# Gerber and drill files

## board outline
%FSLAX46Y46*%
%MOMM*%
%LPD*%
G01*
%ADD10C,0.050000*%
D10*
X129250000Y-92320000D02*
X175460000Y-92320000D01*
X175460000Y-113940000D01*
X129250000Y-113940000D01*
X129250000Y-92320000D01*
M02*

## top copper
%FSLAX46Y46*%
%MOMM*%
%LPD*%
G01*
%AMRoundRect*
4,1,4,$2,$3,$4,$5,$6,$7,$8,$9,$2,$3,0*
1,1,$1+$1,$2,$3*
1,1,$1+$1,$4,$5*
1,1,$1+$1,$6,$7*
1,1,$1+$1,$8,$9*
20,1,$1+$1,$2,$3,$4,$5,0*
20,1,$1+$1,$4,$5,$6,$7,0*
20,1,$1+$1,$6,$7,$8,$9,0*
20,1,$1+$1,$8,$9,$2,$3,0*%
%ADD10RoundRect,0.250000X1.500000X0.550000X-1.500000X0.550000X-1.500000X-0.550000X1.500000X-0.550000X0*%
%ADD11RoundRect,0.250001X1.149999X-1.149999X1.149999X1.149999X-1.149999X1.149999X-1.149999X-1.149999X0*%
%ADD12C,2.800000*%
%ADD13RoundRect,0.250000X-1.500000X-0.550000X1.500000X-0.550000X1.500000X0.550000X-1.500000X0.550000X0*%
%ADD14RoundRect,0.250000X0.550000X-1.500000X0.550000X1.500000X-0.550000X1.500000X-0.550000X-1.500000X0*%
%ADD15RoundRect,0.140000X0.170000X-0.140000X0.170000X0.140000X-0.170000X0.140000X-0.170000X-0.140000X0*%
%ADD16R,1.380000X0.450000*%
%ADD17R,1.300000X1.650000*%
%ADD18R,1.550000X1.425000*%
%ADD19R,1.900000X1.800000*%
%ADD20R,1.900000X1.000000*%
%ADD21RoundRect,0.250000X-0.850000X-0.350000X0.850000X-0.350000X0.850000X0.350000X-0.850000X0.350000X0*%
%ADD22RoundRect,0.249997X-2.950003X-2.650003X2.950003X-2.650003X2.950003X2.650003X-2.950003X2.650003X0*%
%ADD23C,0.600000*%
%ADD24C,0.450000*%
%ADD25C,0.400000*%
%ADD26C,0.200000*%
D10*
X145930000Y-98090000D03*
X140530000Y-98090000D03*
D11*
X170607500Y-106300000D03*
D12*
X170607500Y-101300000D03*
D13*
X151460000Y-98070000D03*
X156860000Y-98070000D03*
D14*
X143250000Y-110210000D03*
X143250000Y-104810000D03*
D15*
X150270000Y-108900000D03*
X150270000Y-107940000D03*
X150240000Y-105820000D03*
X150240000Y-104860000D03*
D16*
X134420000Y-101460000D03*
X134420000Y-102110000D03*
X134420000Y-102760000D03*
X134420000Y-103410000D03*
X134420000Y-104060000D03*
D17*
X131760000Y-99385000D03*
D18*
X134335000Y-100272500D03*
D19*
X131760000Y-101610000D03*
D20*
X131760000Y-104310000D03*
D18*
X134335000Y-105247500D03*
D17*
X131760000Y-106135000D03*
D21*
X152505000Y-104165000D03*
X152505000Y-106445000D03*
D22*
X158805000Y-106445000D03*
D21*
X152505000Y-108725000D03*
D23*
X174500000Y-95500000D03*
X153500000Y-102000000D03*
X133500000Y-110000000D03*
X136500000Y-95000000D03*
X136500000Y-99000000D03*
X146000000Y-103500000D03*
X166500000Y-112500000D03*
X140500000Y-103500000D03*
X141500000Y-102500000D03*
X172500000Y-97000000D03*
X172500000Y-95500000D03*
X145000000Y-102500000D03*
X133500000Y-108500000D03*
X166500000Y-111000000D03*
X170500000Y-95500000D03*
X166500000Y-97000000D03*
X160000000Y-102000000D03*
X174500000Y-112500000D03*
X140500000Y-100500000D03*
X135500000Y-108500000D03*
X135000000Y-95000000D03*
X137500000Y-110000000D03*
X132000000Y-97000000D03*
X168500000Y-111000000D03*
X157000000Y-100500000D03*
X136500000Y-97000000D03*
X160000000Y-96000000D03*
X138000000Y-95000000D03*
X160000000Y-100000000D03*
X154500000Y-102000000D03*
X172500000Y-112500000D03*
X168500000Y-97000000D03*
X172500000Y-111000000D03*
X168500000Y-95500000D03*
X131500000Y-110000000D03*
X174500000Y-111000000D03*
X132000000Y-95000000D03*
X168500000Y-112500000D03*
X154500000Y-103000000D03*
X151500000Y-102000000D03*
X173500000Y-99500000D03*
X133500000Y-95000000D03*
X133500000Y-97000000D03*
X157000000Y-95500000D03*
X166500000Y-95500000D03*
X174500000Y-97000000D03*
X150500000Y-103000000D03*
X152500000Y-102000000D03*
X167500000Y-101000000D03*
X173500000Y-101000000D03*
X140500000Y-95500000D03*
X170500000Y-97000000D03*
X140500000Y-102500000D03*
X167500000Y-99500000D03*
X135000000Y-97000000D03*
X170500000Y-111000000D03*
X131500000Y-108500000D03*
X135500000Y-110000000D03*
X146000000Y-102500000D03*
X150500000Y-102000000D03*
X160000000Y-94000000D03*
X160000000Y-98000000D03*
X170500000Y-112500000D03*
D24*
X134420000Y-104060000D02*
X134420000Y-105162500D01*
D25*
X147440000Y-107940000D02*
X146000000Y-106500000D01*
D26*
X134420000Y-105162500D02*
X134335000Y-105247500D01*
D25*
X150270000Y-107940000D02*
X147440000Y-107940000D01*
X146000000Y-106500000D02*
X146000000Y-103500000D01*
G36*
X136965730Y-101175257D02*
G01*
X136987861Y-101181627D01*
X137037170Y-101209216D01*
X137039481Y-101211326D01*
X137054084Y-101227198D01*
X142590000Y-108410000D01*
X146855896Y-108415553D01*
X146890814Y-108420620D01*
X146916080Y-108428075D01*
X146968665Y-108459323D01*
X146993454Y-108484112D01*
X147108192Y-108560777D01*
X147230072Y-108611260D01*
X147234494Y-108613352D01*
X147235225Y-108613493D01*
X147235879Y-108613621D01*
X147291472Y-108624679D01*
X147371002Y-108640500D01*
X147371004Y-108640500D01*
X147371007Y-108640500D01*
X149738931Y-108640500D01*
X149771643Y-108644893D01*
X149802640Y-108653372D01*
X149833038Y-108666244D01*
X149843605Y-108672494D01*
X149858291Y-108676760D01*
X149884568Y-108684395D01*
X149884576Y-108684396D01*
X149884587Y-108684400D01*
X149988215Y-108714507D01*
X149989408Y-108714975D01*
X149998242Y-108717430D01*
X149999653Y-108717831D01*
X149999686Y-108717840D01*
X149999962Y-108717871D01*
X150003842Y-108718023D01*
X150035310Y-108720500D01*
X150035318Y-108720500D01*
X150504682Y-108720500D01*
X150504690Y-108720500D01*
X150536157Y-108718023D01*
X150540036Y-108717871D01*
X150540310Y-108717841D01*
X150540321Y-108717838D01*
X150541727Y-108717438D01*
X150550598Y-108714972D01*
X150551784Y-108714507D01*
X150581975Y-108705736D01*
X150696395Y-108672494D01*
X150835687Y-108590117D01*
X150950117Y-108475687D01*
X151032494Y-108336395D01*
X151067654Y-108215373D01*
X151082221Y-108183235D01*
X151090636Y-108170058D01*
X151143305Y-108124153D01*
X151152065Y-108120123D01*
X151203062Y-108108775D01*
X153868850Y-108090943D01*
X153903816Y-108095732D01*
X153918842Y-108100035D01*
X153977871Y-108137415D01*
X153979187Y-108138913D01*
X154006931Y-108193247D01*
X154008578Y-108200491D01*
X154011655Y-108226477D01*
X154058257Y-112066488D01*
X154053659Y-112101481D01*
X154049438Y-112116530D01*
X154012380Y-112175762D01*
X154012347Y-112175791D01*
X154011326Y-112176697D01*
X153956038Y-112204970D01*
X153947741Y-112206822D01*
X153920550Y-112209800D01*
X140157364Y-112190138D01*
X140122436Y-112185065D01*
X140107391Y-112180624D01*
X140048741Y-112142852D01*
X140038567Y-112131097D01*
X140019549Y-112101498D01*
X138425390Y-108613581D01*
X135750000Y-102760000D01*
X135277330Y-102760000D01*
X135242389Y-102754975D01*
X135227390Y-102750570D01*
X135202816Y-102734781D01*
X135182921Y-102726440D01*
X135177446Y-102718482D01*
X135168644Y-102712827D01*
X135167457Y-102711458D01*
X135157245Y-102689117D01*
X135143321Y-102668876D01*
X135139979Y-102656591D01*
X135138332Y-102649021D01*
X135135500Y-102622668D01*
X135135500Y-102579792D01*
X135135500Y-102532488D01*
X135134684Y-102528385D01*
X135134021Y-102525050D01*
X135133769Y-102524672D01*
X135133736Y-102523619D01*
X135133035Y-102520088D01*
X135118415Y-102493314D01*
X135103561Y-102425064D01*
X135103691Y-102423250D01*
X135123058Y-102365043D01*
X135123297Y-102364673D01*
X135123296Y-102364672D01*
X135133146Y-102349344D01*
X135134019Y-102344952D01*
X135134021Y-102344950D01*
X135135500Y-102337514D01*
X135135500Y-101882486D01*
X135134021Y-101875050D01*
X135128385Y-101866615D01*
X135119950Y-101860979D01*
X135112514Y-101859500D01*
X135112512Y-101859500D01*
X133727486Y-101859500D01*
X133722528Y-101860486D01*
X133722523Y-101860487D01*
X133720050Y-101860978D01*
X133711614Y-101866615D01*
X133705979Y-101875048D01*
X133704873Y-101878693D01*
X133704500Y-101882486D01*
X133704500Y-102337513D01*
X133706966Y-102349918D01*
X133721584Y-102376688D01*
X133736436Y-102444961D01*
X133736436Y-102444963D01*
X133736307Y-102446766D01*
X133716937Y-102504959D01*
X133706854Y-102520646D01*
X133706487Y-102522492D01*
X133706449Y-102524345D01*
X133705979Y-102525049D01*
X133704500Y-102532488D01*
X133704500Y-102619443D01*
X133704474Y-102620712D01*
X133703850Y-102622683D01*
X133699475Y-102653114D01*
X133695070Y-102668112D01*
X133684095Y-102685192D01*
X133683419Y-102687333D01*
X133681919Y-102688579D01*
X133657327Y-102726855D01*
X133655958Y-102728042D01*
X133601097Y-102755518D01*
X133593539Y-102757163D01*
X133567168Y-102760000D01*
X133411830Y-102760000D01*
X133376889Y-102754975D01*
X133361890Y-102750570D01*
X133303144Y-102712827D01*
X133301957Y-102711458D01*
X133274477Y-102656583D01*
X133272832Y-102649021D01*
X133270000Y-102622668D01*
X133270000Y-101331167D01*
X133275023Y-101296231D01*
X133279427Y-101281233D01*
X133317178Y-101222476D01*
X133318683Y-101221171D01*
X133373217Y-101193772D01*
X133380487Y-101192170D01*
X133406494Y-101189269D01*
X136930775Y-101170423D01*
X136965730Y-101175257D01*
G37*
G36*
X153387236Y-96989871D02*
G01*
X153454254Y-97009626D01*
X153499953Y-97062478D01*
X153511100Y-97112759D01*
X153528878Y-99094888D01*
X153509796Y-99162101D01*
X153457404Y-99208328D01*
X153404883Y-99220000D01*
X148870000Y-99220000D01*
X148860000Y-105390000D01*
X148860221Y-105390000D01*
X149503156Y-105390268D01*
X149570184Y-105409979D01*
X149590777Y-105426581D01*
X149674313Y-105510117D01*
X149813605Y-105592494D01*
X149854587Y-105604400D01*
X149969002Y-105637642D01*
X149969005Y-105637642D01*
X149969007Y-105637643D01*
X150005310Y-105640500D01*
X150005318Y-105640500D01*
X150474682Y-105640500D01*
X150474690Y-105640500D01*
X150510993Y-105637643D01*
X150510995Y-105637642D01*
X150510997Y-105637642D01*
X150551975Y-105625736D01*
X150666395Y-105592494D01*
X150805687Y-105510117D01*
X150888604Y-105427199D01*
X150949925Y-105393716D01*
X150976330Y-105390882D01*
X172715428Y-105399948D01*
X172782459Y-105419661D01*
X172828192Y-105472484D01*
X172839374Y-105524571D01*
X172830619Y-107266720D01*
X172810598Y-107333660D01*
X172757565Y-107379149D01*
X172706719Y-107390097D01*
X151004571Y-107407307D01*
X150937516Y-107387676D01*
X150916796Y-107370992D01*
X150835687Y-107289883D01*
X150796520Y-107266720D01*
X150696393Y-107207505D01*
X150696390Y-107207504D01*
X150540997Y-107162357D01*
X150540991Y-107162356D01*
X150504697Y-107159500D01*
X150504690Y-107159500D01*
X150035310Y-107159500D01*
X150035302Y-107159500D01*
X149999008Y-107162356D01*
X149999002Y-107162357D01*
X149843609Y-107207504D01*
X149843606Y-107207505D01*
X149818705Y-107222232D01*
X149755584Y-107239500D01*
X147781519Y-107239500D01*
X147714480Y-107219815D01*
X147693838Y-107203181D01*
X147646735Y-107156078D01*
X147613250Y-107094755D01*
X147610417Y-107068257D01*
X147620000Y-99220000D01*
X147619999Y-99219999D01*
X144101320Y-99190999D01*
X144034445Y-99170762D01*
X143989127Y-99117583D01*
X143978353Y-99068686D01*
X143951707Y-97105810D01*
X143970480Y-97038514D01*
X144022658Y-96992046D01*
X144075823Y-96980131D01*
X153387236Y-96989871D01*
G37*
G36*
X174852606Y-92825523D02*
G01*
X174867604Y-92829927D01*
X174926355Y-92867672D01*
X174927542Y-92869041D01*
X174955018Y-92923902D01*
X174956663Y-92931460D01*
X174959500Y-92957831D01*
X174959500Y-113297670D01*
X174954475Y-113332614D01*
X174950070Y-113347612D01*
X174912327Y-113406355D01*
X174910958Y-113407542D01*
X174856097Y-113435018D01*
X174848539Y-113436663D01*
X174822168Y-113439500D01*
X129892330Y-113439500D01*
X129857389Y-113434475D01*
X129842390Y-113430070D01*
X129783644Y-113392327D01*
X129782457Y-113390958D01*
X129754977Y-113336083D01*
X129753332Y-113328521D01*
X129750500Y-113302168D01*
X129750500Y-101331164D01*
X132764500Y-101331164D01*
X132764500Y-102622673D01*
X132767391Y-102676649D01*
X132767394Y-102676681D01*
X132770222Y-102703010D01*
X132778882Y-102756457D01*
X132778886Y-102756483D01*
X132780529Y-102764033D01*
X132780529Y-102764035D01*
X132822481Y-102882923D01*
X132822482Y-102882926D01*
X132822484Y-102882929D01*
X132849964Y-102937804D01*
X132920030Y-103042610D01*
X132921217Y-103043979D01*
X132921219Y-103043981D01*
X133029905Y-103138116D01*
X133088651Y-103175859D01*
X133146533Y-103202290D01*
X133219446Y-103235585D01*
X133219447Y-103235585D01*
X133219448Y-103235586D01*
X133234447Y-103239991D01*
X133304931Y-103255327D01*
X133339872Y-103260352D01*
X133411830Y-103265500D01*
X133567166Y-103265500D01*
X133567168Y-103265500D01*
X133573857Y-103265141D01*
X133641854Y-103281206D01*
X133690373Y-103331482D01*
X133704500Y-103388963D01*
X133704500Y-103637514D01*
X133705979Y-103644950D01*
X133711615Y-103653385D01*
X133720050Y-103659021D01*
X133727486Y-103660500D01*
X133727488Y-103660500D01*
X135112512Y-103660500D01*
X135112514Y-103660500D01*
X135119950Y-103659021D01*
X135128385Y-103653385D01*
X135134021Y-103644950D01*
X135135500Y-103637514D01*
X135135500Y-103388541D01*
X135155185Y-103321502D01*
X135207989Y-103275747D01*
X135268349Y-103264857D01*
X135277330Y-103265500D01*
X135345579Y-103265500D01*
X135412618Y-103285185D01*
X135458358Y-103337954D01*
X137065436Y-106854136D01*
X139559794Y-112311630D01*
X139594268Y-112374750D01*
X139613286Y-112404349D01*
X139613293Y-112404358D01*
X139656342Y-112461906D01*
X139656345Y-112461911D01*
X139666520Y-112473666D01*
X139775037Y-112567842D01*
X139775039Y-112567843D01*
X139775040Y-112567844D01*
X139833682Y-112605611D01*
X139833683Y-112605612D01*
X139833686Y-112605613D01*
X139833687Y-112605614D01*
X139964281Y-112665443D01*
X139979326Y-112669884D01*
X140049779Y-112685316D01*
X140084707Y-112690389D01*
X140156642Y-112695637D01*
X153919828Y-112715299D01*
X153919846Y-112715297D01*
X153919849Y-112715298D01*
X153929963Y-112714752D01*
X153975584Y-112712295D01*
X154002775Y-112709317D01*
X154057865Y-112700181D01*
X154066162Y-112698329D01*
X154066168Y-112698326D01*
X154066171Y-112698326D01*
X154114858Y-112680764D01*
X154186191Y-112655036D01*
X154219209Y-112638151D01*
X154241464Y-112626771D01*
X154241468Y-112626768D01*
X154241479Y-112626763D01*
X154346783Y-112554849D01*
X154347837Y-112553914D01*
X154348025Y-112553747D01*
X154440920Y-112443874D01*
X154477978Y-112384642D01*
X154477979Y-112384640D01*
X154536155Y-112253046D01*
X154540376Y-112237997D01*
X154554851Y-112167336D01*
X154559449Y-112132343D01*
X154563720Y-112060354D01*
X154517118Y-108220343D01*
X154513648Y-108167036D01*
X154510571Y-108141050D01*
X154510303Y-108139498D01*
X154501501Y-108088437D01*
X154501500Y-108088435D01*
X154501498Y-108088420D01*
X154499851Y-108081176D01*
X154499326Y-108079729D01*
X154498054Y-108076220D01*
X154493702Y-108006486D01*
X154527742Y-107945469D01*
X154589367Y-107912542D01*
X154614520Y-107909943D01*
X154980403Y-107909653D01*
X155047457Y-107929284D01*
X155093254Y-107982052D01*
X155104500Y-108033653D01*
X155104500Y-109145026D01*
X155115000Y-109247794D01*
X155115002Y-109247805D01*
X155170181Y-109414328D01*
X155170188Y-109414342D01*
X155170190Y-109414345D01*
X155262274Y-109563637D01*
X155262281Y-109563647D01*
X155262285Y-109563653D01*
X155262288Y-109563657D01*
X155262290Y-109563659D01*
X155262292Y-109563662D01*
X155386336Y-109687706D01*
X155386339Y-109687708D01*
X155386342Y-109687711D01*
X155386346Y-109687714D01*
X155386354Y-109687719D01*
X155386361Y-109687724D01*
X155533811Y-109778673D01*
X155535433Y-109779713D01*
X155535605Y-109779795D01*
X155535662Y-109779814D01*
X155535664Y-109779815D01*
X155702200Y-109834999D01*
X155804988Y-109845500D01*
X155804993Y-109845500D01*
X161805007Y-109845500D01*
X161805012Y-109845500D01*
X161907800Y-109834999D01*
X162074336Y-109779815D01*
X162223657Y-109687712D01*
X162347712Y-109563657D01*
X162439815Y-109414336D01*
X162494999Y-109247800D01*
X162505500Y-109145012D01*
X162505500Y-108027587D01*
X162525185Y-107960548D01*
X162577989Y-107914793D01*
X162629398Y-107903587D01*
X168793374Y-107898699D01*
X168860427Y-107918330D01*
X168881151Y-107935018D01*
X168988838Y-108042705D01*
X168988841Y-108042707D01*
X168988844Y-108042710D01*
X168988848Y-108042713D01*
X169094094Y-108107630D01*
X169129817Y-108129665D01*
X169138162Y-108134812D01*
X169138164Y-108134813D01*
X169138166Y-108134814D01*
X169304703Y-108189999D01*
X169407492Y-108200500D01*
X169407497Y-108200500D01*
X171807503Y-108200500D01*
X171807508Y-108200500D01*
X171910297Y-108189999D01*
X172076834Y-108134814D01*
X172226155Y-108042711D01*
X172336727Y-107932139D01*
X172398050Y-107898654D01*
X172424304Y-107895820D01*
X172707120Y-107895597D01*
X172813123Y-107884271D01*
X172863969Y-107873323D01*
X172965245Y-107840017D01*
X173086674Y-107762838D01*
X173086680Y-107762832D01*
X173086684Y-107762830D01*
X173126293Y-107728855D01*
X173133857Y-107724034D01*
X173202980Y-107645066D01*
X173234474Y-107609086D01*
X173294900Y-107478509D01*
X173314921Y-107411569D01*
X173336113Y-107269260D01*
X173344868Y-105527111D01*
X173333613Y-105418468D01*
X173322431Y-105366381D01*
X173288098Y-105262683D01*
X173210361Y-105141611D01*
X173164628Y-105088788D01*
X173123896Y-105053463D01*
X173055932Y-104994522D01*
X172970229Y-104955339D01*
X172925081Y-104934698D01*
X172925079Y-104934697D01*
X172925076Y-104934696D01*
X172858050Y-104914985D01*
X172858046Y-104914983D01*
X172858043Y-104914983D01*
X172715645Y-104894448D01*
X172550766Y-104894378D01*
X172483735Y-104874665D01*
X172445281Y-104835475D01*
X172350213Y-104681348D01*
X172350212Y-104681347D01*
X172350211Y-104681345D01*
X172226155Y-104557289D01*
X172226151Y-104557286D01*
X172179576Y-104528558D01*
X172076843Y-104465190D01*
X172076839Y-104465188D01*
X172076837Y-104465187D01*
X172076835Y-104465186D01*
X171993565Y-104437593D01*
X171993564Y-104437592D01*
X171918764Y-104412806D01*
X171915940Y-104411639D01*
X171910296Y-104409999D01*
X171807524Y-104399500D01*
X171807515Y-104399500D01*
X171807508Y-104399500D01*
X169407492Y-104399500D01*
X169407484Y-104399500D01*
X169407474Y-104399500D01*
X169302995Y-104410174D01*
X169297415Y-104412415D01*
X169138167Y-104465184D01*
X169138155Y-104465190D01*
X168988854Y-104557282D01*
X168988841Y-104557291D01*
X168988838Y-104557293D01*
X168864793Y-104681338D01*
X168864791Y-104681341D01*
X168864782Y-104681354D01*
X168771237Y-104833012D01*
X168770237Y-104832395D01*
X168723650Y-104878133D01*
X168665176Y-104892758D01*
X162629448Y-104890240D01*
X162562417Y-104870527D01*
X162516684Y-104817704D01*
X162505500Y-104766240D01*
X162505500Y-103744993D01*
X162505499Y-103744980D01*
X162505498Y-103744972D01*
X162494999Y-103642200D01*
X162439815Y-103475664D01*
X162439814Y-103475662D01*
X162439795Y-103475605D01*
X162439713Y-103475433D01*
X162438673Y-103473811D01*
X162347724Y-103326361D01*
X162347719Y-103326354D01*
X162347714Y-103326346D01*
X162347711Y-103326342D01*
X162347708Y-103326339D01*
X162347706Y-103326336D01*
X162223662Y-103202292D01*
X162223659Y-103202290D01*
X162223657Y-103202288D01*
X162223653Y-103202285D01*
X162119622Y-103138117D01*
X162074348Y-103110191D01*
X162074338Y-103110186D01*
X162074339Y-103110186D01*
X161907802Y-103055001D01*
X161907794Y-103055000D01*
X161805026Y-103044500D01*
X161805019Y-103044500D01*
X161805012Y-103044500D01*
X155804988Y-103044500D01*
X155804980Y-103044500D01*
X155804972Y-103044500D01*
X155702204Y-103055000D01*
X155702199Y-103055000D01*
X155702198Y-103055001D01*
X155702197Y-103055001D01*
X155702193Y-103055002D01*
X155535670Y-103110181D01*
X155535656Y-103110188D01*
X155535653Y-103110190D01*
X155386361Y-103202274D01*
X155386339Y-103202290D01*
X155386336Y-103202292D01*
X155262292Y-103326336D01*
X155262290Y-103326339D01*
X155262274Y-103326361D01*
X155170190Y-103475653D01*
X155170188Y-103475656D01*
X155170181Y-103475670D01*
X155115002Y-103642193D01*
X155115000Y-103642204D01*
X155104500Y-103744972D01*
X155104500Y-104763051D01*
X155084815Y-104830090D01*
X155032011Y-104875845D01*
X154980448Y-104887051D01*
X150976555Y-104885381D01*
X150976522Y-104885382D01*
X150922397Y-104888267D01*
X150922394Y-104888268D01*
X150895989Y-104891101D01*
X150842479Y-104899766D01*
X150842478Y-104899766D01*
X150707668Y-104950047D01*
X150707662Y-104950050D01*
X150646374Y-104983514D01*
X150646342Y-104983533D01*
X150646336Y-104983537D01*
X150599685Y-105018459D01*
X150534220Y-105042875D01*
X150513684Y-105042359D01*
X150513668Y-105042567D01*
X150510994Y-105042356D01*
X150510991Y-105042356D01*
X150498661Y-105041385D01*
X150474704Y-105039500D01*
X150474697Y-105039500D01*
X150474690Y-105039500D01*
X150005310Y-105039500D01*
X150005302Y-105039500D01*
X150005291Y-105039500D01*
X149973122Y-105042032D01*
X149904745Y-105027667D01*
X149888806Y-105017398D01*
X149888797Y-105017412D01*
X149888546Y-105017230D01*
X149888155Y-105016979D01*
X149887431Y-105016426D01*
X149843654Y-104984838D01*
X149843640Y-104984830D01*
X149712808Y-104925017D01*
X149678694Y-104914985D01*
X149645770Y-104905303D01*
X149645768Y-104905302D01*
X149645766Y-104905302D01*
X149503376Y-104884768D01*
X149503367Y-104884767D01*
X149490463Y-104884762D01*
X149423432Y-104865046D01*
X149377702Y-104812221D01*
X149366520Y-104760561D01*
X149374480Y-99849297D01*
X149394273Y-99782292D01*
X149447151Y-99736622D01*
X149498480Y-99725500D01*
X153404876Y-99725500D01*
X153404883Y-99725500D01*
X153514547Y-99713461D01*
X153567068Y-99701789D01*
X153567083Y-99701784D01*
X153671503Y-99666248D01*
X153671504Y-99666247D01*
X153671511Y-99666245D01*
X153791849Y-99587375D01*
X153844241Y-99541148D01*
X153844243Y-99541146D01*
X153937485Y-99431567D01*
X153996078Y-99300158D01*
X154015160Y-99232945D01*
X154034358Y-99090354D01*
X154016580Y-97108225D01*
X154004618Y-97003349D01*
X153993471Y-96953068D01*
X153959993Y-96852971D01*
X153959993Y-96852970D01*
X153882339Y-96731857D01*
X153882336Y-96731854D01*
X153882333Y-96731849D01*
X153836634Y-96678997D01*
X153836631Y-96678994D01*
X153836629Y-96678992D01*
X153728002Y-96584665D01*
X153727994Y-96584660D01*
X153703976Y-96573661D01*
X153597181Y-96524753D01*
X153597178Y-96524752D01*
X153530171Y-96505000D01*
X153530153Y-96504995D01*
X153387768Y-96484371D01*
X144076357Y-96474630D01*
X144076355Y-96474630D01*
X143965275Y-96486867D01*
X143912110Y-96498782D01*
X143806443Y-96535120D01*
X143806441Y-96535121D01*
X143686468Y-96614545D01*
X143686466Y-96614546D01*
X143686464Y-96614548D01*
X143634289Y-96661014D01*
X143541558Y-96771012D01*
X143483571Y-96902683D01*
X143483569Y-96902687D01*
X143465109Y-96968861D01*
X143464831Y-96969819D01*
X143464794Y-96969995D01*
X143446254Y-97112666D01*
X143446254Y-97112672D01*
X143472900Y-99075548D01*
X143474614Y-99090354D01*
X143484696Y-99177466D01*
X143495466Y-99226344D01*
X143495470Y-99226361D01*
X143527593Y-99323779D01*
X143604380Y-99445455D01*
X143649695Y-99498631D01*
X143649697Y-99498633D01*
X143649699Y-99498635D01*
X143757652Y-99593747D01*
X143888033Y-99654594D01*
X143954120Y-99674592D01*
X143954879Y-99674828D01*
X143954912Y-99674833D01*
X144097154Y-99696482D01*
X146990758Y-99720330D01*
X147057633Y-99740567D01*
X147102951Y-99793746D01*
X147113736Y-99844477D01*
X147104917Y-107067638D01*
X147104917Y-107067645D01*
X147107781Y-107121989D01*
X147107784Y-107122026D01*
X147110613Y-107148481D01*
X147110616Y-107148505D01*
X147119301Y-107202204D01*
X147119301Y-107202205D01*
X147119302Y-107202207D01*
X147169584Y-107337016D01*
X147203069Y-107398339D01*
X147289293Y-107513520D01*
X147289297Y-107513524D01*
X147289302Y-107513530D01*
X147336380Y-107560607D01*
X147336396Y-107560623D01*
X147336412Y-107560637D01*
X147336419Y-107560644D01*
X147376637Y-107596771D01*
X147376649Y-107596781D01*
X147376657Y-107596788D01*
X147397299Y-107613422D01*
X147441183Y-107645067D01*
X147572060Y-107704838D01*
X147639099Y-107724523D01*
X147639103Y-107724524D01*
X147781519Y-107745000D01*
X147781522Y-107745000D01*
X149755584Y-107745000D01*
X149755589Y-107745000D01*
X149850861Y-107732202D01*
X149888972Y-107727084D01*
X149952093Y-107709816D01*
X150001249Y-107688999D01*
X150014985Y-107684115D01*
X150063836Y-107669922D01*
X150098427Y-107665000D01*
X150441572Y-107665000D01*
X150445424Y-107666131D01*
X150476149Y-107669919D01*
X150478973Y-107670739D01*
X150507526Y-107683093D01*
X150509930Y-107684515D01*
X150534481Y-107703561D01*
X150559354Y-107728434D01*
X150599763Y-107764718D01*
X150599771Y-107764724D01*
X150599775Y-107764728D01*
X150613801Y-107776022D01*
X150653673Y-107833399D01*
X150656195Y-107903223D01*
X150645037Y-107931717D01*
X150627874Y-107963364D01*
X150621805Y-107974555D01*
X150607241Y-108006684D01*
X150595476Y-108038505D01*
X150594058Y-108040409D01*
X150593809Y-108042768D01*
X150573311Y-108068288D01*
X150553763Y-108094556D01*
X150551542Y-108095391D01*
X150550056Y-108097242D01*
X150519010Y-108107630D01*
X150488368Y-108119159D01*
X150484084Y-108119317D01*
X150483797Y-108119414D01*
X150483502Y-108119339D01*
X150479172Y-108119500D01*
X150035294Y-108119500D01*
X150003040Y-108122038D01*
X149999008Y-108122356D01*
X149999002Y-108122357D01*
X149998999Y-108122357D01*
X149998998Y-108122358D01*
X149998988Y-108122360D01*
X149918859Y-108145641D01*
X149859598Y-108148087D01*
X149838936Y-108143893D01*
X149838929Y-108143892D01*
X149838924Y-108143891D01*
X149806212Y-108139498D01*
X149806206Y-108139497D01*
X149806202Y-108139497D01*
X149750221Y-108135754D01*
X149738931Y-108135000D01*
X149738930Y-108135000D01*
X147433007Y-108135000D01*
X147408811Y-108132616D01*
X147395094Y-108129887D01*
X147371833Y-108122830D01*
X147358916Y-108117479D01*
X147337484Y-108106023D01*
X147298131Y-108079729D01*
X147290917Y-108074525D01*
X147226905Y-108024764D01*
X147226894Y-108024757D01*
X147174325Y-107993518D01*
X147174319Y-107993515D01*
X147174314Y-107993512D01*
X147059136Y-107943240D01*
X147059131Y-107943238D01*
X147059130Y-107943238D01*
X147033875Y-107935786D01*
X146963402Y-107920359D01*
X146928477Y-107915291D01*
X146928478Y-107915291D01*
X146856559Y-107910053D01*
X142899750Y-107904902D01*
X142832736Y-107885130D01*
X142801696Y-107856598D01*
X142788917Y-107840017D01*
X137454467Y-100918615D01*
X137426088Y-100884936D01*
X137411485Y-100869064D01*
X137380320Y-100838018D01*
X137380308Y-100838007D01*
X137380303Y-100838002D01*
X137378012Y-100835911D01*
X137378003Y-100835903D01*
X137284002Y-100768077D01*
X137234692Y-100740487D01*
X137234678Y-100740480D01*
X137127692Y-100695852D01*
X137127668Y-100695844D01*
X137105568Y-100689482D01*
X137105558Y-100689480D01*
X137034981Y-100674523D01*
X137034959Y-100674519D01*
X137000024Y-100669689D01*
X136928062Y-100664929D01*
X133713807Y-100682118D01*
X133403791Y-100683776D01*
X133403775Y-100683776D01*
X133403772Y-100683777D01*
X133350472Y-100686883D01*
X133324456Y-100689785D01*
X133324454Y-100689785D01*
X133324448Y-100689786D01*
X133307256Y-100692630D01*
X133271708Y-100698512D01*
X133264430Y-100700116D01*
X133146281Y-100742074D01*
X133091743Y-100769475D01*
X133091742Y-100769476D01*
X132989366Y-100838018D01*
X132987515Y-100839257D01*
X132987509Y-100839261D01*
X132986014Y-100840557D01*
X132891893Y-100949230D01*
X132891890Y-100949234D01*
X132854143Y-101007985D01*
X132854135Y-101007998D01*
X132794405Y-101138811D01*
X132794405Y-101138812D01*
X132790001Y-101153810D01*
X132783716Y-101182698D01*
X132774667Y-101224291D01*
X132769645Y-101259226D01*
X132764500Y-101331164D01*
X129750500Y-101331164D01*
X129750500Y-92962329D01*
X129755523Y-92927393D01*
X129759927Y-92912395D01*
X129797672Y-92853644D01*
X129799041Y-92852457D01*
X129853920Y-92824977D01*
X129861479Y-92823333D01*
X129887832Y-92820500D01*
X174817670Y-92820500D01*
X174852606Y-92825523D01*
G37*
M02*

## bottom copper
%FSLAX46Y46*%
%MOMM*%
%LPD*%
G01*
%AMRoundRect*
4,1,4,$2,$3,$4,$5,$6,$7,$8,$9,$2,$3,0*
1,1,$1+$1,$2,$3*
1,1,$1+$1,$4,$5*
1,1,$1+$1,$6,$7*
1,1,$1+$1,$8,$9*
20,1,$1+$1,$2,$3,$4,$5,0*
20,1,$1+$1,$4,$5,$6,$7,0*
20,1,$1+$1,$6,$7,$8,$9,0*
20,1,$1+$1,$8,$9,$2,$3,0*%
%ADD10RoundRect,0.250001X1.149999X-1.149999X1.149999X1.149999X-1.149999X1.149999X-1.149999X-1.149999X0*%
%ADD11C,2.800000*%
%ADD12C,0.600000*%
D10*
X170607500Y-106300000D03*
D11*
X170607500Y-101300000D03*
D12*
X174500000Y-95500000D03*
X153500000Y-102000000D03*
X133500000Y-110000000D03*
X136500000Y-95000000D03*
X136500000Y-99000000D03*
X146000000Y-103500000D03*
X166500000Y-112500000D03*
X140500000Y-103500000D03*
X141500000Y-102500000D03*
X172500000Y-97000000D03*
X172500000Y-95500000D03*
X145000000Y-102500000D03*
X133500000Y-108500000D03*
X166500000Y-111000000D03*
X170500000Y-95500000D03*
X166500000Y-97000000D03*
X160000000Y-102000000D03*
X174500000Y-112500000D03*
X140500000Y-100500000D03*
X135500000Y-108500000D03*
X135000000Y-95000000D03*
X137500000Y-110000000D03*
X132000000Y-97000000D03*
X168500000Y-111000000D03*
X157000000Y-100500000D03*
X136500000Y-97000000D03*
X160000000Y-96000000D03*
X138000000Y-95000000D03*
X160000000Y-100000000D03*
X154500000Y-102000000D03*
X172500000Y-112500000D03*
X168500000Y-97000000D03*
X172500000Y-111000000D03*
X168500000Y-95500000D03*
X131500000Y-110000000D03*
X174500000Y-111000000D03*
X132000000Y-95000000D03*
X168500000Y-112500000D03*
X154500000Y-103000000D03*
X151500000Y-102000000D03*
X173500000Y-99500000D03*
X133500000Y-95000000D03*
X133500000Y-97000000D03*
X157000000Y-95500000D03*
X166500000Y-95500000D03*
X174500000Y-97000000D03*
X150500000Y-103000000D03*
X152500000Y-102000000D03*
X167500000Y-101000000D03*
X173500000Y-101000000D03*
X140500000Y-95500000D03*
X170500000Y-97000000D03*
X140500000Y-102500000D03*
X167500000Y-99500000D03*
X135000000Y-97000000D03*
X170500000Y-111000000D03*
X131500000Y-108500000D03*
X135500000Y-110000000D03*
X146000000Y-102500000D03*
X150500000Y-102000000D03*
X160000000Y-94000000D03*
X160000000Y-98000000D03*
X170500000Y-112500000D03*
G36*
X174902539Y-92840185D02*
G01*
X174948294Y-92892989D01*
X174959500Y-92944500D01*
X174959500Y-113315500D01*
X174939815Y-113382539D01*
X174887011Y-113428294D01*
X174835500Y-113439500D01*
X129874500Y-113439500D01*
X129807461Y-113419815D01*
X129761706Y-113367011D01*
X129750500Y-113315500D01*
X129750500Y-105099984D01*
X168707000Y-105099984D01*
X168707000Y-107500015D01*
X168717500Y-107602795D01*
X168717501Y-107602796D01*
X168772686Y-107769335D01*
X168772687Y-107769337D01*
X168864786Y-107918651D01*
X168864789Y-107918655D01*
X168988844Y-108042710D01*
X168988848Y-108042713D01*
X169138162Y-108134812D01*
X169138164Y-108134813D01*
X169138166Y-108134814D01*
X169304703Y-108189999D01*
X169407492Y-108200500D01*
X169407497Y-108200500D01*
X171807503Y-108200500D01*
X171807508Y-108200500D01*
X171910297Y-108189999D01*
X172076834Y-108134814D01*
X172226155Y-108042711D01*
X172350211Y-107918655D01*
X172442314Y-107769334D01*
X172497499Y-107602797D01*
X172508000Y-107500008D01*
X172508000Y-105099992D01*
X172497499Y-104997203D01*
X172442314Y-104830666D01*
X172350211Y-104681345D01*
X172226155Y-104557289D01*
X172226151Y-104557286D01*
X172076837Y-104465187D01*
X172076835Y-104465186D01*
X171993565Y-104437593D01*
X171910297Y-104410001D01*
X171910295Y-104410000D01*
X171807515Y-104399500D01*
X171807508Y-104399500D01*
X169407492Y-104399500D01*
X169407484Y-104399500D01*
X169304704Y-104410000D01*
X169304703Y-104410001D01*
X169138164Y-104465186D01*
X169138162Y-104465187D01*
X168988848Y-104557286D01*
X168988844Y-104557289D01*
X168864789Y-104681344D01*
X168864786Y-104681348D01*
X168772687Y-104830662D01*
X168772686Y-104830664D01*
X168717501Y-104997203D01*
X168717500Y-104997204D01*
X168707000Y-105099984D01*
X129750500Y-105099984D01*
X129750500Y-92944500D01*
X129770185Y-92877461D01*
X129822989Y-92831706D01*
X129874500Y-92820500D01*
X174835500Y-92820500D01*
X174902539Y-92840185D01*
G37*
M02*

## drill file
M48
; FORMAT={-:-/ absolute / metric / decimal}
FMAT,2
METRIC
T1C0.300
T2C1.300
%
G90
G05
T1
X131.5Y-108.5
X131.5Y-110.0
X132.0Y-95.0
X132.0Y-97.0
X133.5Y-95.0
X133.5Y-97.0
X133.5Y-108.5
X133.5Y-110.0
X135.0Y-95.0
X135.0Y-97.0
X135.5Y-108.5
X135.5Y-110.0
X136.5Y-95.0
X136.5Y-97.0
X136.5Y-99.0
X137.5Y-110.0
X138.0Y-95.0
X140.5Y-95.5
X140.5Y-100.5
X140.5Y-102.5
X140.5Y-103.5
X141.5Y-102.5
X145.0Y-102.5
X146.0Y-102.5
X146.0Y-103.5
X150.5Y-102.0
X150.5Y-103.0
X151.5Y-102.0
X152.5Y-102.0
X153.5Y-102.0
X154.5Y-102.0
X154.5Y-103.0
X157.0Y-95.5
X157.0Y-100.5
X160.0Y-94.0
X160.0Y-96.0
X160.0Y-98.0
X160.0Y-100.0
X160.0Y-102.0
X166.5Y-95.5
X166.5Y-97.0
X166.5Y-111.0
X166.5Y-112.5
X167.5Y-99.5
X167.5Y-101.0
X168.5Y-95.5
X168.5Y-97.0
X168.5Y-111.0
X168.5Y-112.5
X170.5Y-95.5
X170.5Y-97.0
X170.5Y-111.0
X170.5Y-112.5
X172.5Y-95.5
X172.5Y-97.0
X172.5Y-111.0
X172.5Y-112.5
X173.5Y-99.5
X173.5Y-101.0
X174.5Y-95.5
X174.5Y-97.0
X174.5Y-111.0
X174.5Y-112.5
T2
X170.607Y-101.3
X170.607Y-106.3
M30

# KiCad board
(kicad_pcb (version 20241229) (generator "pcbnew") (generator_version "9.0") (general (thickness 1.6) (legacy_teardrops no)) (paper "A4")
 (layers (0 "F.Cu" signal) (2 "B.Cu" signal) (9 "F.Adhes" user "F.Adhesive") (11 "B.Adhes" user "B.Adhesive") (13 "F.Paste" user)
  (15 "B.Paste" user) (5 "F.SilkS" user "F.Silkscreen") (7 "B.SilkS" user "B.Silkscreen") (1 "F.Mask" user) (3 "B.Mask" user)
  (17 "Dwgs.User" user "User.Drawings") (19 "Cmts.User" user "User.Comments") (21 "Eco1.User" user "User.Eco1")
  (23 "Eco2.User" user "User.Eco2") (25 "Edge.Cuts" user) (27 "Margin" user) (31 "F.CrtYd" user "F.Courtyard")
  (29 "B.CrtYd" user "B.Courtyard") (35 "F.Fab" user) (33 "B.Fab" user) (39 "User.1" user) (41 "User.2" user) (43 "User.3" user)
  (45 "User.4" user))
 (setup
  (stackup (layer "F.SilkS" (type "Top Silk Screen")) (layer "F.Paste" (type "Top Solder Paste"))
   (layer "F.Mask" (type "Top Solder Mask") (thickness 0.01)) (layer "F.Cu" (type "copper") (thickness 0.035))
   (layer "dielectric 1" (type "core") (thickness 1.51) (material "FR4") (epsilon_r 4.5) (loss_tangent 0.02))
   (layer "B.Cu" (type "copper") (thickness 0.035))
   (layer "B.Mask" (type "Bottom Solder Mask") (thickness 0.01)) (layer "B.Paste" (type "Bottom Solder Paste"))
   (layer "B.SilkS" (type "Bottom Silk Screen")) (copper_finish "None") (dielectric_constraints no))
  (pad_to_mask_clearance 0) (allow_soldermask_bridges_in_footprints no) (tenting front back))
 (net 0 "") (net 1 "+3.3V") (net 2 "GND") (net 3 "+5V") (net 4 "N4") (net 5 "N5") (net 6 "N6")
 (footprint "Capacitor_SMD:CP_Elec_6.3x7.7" (layer "F.Cu") (at 143.23 98.09 180)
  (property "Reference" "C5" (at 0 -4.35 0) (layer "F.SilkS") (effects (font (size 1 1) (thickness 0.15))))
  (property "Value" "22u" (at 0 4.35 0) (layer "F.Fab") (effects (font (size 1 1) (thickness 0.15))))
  (pad "1" smd roundrect (at -2.7 0 180) (size 3.5 1.6) (layers "F.Cu" "F.Mask" "F.Paste") (roundrect_rratio 0.15625) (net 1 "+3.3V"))
  (pad "2" smd roundrect (at 2.7 0 180) (size 3.5 1.6) (layers "F.Cu" "F.Mask" "F.Paste") (roundrect_rratio 0.15625) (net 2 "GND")))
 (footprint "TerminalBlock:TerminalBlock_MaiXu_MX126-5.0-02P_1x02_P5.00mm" (layer "F.Cu") (at 170.6075 106.3 90)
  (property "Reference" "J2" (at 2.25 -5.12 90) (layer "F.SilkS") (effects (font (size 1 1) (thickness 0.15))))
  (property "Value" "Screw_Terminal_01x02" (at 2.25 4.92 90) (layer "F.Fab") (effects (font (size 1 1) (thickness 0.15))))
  (pad "1" thru_hole roundrect (at 0 0 90) (size 2.8 2.8) (drill 1.3) (layers "*.Cu" "*.Mask") (remove_unused_layers no)
   (roundrect_rratio 0.089286) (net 1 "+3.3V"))
  (pad "2" thru_hole circle (at 5 0 90) (size 2.8 2.8) (drill 1.3) (layers "*.Cu" "*.Mask") (remove_unused_layers no) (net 2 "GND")))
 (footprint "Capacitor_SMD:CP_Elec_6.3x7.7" (layer "F.Cu") (at 154.16 98.07)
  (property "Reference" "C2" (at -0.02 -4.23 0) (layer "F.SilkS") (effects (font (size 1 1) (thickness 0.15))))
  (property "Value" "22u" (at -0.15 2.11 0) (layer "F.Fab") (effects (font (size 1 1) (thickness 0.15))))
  (pad "1" smd roundrect (at -2.7 0) (size 3.5 1.6) (layers "F.Cu" "F.Mask" "F.Paste") (roundrect_rratio 0.15625) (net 1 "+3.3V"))
  (pad "2" smd roundrect (at 2.7 0) (size 3.5 1.6) (layers "F.Cu" "F.Mask" "F.Paste") (roundrect_rratio 0.15625) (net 2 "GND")))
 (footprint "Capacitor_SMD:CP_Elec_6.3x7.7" (layer "F.Cu") (at 143.25 107.51 90)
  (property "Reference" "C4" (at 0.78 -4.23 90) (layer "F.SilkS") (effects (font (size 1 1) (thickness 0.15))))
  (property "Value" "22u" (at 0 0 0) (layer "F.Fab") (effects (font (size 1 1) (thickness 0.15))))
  (pad "1" smd roundrect (at -2.7 0 90) (size 3.5 1.6) (layers "F.Cu" "F.Mask" "F.Paste") (roundrect_rratio 0.15625) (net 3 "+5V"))
  (pad "2" smd roundrect (at 2.7 0 90) (size 3.5 1.6) (layers "F.Cu" "F.Mask" "F.Paste") (roundrect_rratio 0.15625) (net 2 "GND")))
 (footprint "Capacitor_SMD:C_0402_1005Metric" (layer "F.Cu") (at 150.27 108.42 90)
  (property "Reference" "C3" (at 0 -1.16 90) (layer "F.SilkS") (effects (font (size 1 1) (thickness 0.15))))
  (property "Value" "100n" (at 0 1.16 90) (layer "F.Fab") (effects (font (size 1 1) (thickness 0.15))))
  (pad "1" smd roundrect (at -0.48 0 90) (size 0.56 0.62) (layers "F.Cu" "F.Mask" "F.Paste") (roundrect_rratio 0.25) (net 3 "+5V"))
  (pad "2" smd roundrect (at 0.48 0 90) (size 0.56 0.62) (layers "F.Cu" "F.Mask" "F.Paste") (roundrect_rratio 0.25) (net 2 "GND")))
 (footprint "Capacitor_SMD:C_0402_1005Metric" (layer "F.Cu") (at 150.24 105.34 90)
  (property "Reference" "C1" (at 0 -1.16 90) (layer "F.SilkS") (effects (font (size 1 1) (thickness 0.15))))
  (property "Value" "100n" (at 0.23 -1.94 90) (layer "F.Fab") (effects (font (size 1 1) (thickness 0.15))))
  (pad "1" smd roundrect (at -0.48 0 90) (size 0.56 0.62) (layers "F.Cu" "F.Mask" "F.Paste") (roundrect_rratio 0.25) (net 1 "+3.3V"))
  (pad "2" smd roundrect (at 0.48 0 90) (size 0.56 0.62) (layers "F.Cu" "F.Mask" "F.Paste") (roundrect_rratio 0.25) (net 2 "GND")))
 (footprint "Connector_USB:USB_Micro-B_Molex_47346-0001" (layer "F.Cu") (at 132.96 102.76 -90)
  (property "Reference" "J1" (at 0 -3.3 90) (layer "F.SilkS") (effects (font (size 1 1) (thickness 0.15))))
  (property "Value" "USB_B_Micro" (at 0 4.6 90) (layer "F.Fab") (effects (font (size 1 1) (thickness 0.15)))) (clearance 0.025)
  (pad "1" smd rect (at -1.3 -1.46 270) (size 0.45 1.38) (layers "F.Cu" "F.Mask" "F.Paste") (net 3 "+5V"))
  (pad "2" smd rect (at -0.65 -1.46 270) (size 0.45 1.38) (layers "F.Cu" "F.Mask" "F.Paste") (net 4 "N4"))
  (pad "3" smd rect (at 0 -1.46 270) (size 0.45 1.38) (layers "F.Cu" "F.Mask" "F.Paste") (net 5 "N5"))
  (pad "4" smd rect (at 0.65 -1.46 270) (size 0.45 1.38) (layers "F.Cu" "F.Mask" "F.Paste") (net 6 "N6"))
  (pad "5" smd rect (at 1.3 -1.46 270) (size 0.45 1.38) (layers "F.Cu" "F.Mask" "F.Paste") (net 2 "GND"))
  (pad "6" smd rect (at -3.375 1.2 270) (size 1.65 1.3) (layers "F.Cu" "F.Mask" "F.Paste") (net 2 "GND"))
  (pad "6" smd rect (at -2.4875 -1.375 270) (size 1.425 1.55) (layers "F.Cu" "F.Mask" "F.Paste") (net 2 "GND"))
  (pad "6" smd rect (at -1.15 1.2 270) (size 1.8 1.9) (layers "F.Cu" "F.Mask" "F.Paste") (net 2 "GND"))
  (pad "6" smd rect (at 1.55 1.2 270) (size 1 1.9) (layers "F.Cu" "F.Mask" "F.Paste") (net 2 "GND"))
  (pad "6" smd rect (at 2.4875 -1.375 270) (size 1.425 1.55) (layers "F.Cu" "F.Mask" "F.Paste") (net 2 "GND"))
  (pad "6" smd rect (at 3.375 1.2 270) (size 1.65 1.3) (layers "F.Cu" "F.Mask" "F.Paste") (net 2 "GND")))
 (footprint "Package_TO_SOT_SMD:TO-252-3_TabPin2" (layer "F.Cu") (at 157.545 106.445)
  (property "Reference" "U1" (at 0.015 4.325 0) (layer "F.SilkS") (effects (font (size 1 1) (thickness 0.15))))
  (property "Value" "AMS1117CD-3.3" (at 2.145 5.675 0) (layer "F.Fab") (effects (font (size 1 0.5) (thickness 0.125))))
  (pad "" smd roundrect (at -0.415 -1.525) (size 3.05 2.75) (layers "F.Paste") (roundrect_rratio 0.090909))
  (pad "" smd roundrect (at -0.415 1.525) (size 3.05 2.75) (layers "F.Paste") (roundrect_rratio 0.090909))
  (pad "" smd roundrect (at 2.935 -1.525) (size 3.05 2.75) (layers "F.Paste") (roundrect_rratio 0.090909))
  (pad "" smd roundrect (at 2.935 1.525) (size 3.05 2.75) (layers "F.Paste") (roundrect_rratio 0.090909))
  (pad "1" smd roundrect (at -5.04 -2.28) (size 2.2 1.2) (layers "F.Cu" "F.Mask" "F.Paste") (roundrect_rratio 0.208333) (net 2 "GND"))
  (pad "2" smd roundrect (at -5.04 0) (size 2.2 1.2) (layers "F.Cu" "F.Mask" "F.Paste") (roundrect_rratio 0.208333) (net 1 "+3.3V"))
  (pad "2" smd roundrect (at 1.26 0) (size 6.4 5.8) (layers "F.Cu" "F.Mask") (roundrect_rratio 0.043103) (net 1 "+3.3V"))
  (pad "3" smd roundrect (at -5.04 2.28) (size 2.2 1.2) (layers "F.Cu" "F.Mask" "F.Paste") (roundrect_rratio 0.208333) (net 3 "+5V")))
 (gr_rect (start 129.25 92.32) (end 175.46 113.94) (stroke (width 0.05) (type default)) (fill no) (layer "Edge.Cuts"))
 (segment (start 134.42 104.06) (end 134.42 105.1625) (width 0.45) (layer "F.Cu") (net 2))
 (segment (start 147.44 107.94) (end 146 106.5) (width 0.4) (layer "F.Cu") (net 2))
 (segment (start 134.42 105.1625) (end 134.335 105.2475) (width 0.2) (layer "F.Cu") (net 2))
 (segment (start 150.27 107.94) (end 147.44 107.94) (width 0.4) (layer "F.Cu") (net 2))
 (segment (start 146 106.5) (end 146 103.5) (width 0.4) (layer "F.Cu") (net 2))
 (via (at 174.5 95.5) (size 0.6) (drill 0.3) (layers "F.Cu" "B.Cu") (free yes) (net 2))
 (via (at 153.5 102) (size 0.6) (drill 0.3) (layers "F.Cu" "B.Cu") (free yes) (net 2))
 (via (at 133.5 110) (size 0.6) (drill 0.3) (layers "F.Cu" "B.Cu") (free yes) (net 2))
 (via (at 136.5 95) (size 0.6) (drill 0.3) (layers "F.Cu" "B.Cu") (free yes) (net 2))
 (via (at 136.5 99) (size 0.6) (drill 0.3) (layers "F.Cu" "B.Cu") (free yes) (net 2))
 (via (at 146 103.5) (size 0.6) (drill 0.3) (layers "F.Cu" "B.Cu") (free yes) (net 2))
 (via (at 166.5 112.5) (size 0.6) (drill 0.3) (layers "F.Cu" "B.Cu") (free yes) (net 2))
 (via (at 140.5 103.5) (size 0.6) (drill 0.3) (layers "F.Cu" "B.Cu") (free yes) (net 2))
 (via (at 141.5 102.5) (size 0.6) (drill 0.3) (layers "F.Cu" "B.Cu") (free yes) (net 2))
 (via (at 172.5 97) (size 0.6) (drill 0.3) (layers "F.Cu" "B.Cu") (free yes) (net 2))
 (via (at 172.5 95.5) (size 0.6) (drill 0.3) (layers "F.Cu" "B.Cu") (free yes) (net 2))
 (via (at 145 102.5) (size 0.6) (drill 0.3) (layers "F.Cu" "B.Cu") (free yes) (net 2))
 (via (at 133.5 108.5) (size 0.6) (drill 0.3) (layers "F.Cu" "B.Cu") (free yes) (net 2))
 (via (at 166.5 111) (size 0.6) (drill 0.3) (layers "F.Cu" "B.Cu") (free yes) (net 2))
 (via (at 170.5 95.5) (size 0.6) (drill 0.3) (layers "F.Cu" "B.Cu") (free yes) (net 2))
 (via (at 166.5 97) (size 0.6) (drill 0.3) (layers "F.Cu" "B.Cu") (free yes) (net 2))
 (via (at 160 102) (size 0.6) (drill 0.3) (layers "F.Cu" "B.Cu") (free yes) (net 2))
 (via (at 174.5 112.5) (size 0.6) (drill 0.3) (layers "F.Cu" "B.Cu") (free yes) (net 2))
 (via (at 140.5 100.5) (size 0.6) (drill 0.3) (layers "F.Cu" "B.Cu") (free yes) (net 2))
 (via (at 135.5 108.5) (size 0.6) (drill 0.3) (layers "F.Cu" "B.Cu") (free yes) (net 2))
 (via (at 135 95) (size 0.6) (drill 0.3) (layers "F.Cu" "B.Cu") (free yes) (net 2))
 (via (at 137.5 110) (size 0.6) (drill 0.3) (layers "F.Cu" "B.Cu") (free yes) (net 2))
 (via (at 132 97) (size 0.6) (drill 0.3) (layers "F.Cu" "B.Cu") (free yes) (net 2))
 (via (at 168.5 111) (size 0.6) (drill 0.3) (layers "F.Cu" "B.Cu") (free yes) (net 2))
 (via (at 157 100.5) (size 0.6) (drill 0.3) (layers "F.Cu" "B.Cu") (free yes) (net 2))
 (via (at 136.5 97) (size 0.6) (drill 0.3) (layers "F.Cu" "B.Cu") (free yes) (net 2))
 (via (at 160 96) (size 0.6) (drill 0.3) (layers "F.Cu" "B.Cu") (free yes) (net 2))
 (via (at 138 95) (size 0.6) (drill 0.3) (layers "F.Cu" "B.Cu") (free yes) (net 2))
 (via (at 160 100) (size 0.6) (drill 0.3) (layers "F.Cu" "B.Cu") (free yes) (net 2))
 (via (at 154.5 102) (size 0.6) (drill 0.3) (layers "F.Cu" "B.Cu") (free yes) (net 2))
 (via (at 172.5 112.5) (size 0.6) (drill 0.3) (layers "F.Cu" "B.Cu") (free yes) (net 2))
 (via (at 168.5 97) (size 0.6) (drill 0.3) (layers "F.Cu" "B.Cu") (free yes) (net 2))
 (via (at 172.5 111) (size 0.6) (drill 0.3) (layers "F.Cu" "B.Cu") (free yes) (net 2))
 (via (at 168.5 95.5) (size 0.6) (drill 0.3) (layers "F.Cu" "B.Cu") (free yes) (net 2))
 (via (at 131.5 110) (size 0.6) (drill 0.3) (layers "F.Cu" "B.Cu") (free yes) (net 2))
 (via (at 174.5 111) (size 0.6) (drill 0.3) (layers "F.Cu" "B.Cu") (free yes) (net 2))
 (via (at 132 95) (size 0.6) (drill 0.3) (layers "F.Cu" "B.Cu") (free yes) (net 2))
 (via (at 168.5 112.5) (size 0.6) (drill 0.3) (layers "F.Cu" "B.Cu") (free yes) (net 2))
 (via (at 154.5 103) (size 0.6) (drill 0.3) (layers "F.Cu" "B.Cu") (free yes) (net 2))
 (via (at 151.5 102) (size 0.6) (drill 0.3) (layers "F.Cu" "B.Cu") (free yes) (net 2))
 (via (at 173.5 99.5) (size 0.6) (drill 0.3) (layers "F.Cu" "B.Cu") (free yes) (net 2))
 (via (at 133.5 95) (size 0.6) (drill 0.3) (layers "F.Cu" "B.Cu") (free yes) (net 2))
 (via (at 133.5 97) (size 0.6) (drill 0.3) (layers "F.Cu" "B.Cu") (free yes) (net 2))
 (via (at 157 95.5) (size 0.6) (drill 0.3) (layers "F.Cu" "B.Cu") (free yes) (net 2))
 (via (at 166.5 95.5) (size 0.6) (drill 0.3) (layers "F.Cu" "B.Cu") (free yes) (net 2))
 (via (at 174.5 97) (size 0.6) (drill 0.3) (layers "F.Cu" "B.Cu") (free yes) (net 2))
 (via (at 150.5 103) (size 0.6) (drill 0.3) (layers "F.Cu" "B.Cu") (free yes) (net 2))
 (via (at 152.5 102) (size 0.6) (drill 0.3) (layers "F.Cu" "B.Cu") (free yes) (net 2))
 (via (at 167.5 101) (size 0.6) (drill 0.3) (layers "F.Cu" "B.Cu") (free yes) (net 2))
 (via (at 173.5 101) (size 0.6) (drill 0.3) (layers "F.Cu" "B.Cu") (free yes) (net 2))
 (via (at 140.5 95.5) (size 0.6) (drill 0.3) (layers "F.Cu" "B.Cu") (free yes) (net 2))
 (via (at 170.5 97) (size 0.6) (drill 0.3) (layers "F.Cu" "B.Cu") (free yes) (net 2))
 (via (at 140.5 102.5) (size 0.6) (drill 0.3) (layers "F.Cu" "B.Cu") (free yes) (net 2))
 (via (at 167.5 99.5) (size 0.6) (drill 0.3) (layers "F.Cu" "B.Cu") (free yes) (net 2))
 (via (at 135 97) (size 0.6) (drill 0.3) (layers "F.Cu" "B.Cu") (free yes) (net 2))
 (via (at 170.5 111) (size 0.6) (drill 0.3) (layers "F.Cu" "B.Cu") (free yes) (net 2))
 (via (at 131.5 108.5) (size 0.6) (drill 0.3) (layers "F.Cu" "B.Cu") (free yes) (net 2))
 (via (at 135.5 110) (size 0.6) (drill 0.3) (layers "F.Cu" "B.Cu") (free yes) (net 2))
 (via (at 146 102.5) (size 0.6) (drill 0.3) (layers "F.Cu" "B.Cu") (free yes) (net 2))
 (via (at 150.5 102) (size 0.6) (drill 0.3) (layers "F.Cu" "B.Cu") (free yes) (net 2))
 (via (at 160 94) (size 0.6) (drill 0.3) (layers "F.Cu" "B.Cu") (free yes) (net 2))
 (via (at 160 98) (size 0.6) (drill 0.3) (layers "F.Cu" "B.Cu") (free yes) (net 2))
 (via (at 170.5 112.5) (size 0.6) (drill 0.3) (layers "F.Cu" "B.Cu") (free yes) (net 2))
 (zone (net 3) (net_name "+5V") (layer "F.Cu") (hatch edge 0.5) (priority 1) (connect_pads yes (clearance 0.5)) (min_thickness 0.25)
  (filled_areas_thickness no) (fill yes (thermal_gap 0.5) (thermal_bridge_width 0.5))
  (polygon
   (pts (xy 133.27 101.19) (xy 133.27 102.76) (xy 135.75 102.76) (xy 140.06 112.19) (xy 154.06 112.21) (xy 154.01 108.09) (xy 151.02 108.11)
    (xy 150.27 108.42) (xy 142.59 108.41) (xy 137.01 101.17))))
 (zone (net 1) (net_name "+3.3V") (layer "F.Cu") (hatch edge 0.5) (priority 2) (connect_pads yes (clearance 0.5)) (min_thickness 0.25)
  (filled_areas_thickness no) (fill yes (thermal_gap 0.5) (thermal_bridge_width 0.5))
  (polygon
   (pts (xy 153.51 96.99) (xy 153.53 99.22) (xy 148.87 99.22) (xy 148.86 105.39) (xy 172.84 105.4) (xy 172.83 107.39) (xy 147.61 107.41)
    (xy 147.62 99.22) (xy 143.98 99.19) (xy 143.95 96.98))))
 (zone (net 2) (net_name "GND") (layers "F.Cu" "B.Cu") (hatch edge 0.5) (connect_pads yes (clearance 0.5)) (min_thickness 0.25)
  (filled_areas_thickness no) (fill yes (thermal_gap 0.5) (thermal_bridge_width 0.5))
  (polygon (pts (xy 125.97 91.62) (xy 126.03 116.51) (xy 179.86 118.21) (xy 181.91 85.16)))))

